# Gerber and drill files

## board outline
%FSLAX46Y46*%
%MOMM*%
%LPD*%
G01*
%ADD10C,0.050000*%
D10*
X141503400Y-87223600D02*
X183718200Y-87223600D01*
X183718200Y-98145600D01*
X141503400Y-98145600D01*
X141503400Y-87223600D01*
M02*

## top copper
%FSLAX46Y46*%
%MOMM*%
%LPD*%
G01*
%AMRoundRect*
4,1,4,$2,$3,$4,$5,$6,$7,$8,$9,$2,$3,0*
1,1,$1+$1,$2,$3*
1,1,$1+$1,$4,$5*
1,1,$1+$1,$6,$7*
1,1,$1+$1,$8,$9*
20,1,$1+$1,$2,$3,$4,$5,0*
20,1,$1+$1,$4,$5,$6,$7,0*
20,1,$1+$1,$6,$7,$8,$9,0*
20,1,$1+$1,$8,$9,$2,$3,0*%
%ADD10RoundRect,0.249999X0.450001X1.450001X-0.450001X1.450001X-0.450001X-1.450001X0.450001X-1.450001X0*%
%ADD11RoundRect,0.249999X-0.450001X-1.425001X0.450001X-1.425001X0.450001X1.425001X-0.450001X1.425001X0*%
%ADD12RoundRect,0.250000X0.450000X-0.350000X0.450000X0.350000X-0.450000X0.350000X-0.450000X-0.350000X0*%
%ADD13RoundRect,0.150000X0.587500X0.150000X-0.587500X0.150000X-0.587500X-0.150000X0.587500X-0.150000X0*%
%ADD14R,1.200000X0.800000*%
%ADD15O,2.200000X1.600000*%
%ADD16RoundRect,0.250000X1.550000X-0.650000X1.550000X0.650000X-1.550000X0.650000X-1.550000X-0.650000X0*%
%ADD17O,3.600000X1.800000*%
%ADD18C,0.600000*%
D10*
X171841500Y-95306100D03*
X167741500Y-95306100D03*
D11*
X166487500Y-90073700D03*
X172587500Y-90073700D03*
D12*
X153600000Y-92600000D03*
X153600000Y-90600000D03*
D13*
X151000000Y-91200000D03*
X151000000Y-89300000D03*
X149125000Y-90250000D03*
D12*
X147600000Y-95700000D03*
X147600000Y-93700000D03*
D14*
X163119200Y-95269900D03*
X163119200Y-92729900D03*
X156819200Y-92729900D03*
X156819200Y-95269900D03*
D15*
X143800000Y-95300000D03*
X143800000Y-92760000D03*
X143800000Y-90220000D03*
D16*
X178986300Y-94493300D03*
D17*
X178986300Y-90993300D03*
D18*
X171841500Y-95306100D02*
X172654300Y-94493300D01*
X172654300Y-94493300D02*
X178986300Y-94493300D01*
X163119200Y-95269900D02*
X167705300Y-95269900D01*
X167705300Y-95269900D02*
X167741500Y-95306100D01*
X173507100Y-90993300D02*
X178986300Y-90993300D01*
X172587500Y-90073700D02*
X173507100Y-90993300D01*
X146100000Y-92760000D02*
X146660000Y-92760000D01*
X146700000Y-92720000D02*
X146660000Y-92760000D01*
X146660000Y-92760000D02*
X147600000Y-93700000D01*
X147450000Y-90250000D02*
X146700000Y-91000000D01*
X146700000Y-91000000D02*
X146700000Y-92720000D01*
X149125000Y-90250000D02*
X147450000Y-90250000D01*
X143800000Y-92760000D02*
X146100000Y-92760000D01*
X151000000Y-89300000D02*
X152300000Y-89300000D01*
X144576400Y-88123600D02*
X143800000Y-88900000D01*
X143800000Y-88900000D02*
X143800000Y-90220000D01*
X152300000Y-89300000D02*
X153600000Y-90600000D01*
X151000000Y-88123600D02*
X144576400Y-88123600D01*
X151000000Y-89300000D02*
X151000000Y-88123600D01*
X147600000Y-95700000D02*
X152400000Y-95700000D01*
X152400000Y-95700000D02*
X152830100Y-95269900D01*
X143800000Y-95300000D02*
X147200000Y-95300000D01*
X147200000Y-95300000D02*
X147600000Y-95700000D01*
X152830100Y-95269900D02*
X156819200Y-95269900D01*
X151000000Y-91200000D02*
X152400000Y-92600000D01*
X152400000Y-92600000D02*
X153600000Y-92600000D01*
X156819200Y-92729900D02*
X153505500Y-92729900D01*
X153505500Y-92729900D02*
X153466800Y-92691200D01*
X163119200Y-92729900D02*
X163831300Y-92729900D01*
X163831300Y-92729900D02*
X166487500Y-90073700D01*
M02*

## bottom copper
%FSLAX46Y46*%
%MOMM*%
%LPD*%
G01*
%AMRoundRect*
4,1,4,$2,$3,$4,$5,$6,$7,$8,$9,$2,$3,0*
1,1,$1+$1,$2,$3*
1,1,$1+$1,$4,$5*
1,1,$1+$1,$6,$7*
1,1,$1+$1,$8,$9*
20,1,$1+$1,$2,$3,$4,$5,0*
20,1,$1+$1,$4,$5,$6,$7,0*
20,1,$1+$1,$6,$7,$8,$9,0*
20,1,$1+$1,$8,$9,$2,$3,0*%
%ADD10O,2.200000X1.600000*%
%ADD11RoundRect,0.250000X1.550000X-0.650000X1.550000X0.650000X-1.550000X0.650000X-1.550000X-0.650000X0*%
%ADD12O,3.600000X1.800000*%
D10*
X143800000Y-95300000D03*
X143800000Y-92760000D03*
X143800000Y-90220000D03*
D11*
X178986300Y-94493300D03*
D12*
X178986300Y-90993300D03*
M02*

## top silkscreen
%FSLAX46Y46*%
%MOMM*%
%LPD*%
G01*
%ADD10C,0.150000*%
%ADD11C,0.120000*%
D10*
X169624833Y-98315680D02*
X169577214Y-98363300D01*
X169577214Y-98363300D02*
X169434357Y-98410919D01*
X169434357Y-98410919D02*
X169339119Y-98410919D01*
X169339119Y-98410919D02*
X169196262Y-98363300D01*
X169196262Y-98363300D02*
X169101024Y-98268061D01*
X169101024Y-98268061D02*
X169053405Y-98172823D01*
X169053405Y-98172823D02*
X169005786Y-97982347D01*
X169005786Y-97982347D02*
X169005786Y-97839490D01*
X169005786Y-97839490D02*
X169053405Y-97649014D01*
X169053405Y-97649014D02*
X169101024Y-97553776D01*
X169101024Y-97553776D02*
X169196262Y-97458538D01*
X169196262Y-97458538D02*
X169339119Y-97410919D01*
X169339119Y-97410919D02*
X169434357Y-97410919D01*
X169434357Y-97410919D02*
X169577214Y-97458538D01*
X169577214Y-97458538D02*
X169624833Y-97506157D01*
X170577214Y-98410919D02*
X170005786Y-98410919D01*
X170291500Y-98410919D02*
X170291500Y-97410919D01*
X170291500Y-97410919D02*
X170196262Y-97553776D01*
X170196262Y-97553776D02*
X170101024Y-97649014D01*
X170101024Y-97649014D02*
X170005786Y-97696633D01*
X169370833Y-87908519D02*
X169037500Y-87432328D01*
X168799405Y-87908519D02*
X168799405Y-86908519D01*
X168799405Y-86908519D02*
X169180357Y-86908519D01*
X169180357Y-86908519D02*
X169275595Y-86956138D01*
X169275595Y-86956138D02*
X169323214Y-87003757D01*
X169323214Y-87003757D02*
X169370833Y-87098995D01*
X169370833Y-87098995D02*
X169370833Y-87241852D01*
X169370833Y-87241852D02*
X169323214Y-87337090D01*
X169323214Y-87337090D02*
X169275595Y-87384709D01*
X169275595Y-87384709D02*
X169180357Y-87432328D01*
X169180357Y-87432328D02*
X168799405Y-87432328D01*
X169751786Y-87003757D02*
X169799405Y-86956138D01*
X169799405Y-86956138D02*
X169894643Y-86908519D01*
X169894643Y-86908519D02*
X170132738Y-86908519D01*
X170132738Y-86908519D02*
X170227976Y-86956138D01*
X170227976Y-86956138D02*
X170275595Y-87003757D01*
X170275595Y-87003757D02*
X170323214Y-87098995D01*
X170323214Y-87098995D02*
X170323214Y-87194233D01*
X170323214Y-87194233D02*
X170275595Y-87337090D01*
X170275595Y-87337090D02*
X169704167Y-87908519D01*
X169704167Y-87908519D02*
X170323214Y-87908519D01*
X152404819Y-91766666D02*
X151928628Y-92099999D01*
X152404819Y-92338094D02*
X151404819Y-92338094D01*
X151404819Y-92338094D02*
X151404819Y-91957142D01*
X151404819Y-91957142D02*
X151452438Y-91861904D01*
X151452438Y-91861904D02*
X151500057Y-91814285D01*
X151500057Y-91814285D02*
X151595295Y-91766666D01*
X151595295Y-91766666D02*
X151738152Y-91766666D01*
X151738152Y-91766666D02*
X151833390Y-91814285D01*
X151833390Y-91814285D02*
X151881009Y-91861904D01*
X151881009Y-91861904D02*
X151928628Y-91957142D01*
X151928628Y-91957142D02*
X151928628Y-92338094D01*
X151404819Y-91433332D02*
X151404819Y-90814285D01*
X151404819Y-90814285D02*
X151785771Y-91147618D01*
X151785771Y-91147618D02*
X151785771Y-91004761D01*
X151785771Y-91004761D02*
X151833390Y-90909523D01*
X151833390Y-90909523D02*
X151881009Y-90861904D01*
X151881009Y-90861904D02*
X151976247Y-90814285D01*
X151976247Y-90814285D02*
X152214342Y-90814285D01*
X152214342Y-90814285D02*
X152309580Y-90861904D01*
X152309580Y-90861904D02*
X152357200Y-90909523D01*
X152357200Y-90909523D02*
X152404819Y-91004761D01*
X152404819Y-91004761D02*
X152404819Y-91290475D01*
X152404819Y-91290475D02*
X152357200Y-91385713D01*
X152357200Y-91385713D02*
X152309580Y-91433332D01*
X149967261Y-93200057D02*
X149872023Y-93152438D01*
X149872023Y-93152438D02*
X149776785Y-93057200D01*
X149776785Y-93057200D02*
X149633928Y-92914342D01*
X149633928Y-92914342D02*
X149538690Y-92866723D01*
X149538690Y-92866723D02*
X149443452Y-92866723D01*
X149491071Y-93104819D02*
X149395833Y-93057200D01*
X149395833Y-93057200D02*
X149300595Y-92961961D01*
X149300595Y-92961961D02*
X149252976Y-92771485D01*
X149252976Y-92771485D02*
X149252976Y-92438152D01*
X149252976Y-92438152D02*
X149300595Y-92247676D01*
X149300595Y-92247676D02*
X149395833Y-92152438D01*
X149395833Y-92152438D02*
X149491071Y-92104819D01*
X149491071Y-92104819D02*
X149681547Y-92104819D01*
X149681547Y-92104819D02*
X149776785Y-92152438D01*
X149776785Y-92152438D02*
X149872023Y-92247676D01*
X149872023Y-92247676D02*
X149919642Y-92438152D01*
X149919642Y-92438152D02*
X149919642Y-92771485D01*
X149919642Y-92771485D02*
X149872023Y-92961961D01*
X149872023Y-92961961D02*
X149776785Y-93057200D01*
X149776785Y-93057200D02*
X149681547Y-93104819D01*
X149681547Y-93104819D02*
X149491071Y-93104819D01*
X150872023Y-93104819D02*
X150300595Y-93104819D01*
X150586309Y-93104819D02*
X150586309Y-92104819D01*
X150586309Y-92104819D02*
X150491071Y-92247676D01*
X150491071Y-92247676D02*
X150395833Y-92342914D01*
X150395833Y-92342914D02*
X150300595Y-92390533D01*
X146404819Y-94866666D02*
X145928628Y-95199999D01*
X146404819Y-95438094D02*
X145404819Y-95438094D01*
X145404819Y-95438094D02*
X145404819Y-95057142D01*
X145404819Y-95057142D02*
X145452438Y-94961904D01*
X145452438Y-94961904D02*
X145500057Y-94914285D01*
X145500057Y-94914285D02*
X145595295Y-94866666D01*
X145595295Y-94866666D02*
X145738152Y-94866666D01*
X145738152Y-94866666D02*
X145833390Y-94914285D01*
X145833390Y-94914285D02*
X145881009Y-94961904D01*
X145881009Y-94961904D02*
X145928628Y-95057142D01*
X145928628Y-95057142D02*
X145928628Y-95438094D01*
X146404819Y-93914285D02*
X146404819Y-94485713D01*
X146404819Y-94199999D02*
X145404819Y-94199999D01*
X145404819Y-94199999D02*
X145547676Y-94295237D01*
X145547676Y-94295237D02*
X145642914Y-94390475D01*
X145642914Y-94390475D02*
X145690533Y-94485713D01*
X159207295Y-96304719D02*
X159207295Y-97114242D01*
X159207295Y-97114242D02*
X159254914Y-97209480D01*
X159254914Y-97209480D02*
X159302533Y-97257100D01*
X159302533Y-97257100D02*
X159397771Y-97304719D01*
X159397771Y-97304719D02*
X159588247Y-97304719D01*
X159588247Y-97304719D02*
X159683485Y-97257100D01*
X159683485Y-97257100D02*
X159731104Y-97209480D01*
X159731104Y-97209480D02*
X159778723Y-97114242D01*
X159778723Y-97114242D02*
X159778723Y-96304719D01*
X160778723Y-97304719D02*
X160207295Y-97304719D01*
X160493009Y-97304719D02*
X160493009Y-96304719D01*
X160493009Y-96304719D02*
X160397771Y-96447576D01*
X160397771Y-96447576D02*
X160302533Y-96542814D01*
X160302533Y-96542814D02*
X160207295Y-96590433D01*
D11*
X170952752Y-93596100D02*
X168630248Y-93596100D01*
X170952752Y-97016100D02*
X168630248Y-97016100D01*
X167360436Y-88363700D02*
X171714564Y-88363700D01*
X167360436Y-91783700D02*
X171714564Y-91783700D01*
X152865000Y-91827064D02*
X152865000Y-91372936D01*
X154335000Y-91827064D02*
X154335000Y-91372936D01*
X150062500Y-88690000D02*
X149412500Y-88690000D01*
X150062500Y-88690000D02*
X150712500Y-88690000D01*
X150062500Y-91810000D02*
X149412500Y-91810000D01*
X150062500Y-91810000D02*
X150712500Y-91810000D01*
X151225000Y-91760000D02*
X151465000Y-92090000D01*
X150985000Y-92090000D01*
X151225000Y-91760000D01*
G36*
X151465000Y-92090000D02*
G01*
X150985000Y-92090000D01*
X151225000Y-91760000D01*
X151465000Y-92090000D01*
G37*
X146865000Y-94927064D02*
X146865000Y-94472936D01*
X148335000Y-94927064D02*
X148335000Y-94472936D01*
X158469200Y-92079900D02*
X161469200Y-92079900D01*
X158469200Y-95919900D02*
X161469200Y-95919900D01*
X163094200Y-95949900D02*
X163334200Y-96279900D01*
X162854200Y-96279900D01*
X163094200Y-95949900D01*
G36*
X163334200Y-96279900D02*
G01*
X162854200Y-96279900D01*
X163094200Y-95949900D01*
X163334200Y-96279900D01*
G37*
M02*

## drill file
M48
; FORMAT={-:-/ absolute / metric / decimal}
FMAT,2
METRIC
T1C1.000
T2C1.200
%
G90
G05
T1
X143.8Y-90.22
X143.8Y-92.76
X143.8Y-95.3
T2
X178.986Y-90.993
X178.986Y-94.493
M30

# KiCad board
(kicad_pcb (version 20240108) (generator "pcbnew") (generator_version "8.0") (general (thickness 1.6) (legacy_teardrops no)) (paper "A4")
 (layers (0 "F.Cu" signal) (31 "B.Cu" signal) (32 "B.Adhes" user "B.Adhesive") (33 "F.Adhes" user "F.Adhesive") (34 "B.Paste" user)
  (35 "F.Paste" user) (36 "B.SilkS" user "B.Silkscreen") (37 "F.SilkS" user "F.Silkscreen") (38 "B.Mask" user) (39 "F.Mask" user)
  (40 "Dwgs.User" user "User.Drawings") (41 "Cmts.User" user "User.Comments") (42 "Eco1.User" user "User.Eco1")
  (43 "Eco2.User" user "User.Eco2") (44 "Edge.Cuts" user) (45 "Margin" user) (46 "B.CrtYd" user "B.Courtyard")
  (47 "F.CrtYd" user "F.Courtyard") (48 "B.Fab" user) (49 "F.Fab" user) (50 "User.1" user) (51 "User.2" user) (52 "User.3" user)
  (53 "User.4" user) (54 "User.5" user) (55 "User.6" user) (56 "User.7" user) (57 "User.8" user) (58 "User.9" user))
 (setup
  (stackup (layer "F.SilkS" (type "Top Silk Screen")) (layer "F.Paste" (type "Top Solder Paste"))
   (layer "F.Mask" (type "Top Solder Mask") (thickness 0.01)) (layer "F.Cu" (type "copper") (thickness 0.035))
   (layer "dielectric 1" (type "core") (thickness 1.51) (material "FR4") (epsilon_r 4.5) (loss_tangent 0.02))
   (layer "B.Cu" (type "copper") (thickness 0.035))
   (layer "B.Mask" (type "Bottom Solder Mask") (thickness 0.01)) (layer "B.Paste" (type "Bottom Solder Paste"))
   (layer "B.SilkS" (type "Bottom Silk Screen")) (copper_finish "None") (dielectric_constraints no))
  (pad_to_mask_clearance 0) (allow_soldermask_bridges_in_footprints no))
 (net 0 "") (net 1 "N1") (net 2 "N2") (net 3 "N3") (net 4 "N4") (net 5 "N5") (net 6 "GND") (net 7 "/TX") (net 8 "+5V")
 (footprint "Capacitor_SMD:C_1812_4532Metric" (layer "F.Cu") (at 169.7915 95.3061 180)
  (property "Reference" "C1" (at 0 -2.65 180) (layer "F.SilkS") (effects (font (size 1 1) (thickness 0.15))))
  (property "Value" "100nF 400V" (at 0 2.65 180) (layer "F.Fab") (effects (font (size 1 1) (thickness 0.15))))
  (fp_line (start -1.161252 1.71) (end 1.161252 1.71) (stroke (width 0.12) (type solid)) (layer "F.SilkS"))
  (fp_line (start -1.161252 -1.71) (end 1.161252 -1.71) (stroke (width 0.12) (type solid)) (layer "F.SilkS"))
  (pad "1" smd roundrect (at -2.05 0 180) (size 1.4 3.4) (layers "F.Cu" "F.Paste" "F.Mask") (roundrect_rratio 0.178571) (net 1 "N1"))
  (pad "2" smd roundrect (at 2.05 0 180) (size 1.4 3.4) (layers "F.Cu" "F.Paste" "F.Mask") (roundrect_rratio 0.178571) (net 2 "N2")))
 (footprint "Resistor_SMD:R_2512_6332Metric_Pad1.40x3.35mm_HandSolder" (layer "F.Cu") (at 169.5375 90.0737)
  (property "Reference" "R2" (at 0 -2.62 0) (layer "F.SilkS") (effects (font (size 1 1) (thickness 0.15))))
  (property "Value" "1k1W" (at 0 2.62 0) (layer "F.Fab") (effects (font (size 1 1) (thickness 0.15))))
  (fp_line (start -2.177064 -1.71) (end 2.177064 -1.71) (stroke (width 0.12) (type solid)) (layer "F.SilkS"))
  (fp_line (start -2.177064 1.71) (end 2.177064 1.71) (stroke (width 0.12) (type solid)) (layer "F.SilkS"))
  (pad "1" smd roundrect (at -3.05 0) (size 1.4 3.35) (layers "F.Cu" "F.Paste" "F.Mask") (roundrect_rratio 0.178571) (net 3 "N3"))
  (pad "2" smd roundrect (at 3.05 0) (size 1.4 3.35) (layers "F.Cu" "F.Paste" "F.Mask") (roundrect_rratio 0.178571) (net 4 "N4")))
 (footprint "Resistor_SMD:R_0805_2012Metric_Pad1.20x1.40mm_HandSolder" (layer "F.Cu") (at 153.6 91.6 90)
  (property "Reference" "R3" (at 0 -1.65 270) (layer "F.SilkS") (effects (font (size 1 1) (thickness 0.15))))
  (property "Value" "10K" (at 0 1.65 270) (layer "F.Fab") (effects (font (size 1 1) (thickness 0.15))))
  (fp_line (start -0.227064 -0.735) (end 0.227064 -0.735) (stroke (width 0.12) (type solid)) (layer "F.SilkS"))
  (fp_line (start -0.227064 0.735) (end 0.227064 0.735) (stroke (width 0.12) (type solid)) (layer "F.SilkS"))
  (pad "1" smd roundrect (at -1 0 90) (size 1.2 1.4) (layers "F.Cu" "F.Paste" "F.Mask") (roundrect_rratio 0.208333) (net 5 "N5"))
  (pad "2" smd roundrect (at 1 0 90) (size 1.2 1.4) (layers "F.Cu" "F.Paste" "F.Mask") (roundrect_rratio 0.208333) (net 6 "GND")))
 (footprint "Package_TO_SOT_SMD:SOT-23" (layer "F.Cu") (at 150.0625 90.25 180)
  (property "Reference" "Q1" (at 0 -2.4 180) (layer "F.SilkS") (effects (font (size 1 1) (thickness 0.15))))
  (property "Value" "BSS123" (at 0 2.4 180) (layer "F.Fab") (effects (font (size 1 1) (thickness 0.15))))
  (fp_line (start 0 1.56) (end 0.65 1.56) (stroke (width 0.12) (type solid)) (layer "F.SilkS"))
  (fp_line (start 0 1.56) (end -0.65 1.56) (stroke (width 0.12) (type solid)) (layer "F.SilkS"))
  (fp_line (start 0 -1.56) (end 0.65 -1.56) (stroke (width 0.12) (type solid)) (layer "F.SilkS"))
  (fp_line (start 0 -1.56) (end -0.65 -1.56) (stroke (width 0.12) (type solid)) (layer "F.SilkS"))
  (fp_poly
   (pts (xy -1.1625 -1.51) (xy -1.4025 -1.84) (xy -0.9225 -1.84) (xy -1.1625 -1.51)) (stroke (width 0.12) (type solid)) (fill solid)
   (layer "F.SilkS"))
  (pad "1" smd roundrect (at -0.9375 -0.95 180) (size 1.475 0.6) (layers "F.Cu" "F.Paste" "F.Mask") (roundrect_rratio 0.25) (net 5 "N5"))
  (pad "2" smd roundrect (at -0.9375 0.95 180) (size 1.475 0.6) (layers "F.Cu" "F.Paste" "F.Mask") (roundrect_rratio 0.25) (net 6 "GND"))
  (pad "3" smd roundrect (at 0.9375 0 180) (size 1.475 0.6) (layers "F.Cu" "F.Paste" "F.Mask") (roundrect_rratio 0.25) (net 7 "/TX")))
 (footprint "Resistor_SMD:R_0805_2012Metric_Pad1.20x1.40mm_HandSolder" (layer "F.Cu") (at 147.6 94.7 90)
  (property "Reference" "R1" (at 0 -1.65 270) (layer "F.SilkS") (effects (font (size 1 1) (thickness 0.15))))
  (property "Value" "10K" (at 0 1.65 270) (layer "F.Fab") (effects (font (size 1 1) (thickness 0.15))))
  (fp_line (start -0.227064 -0.735) (end 0.227064 -0.735) (stroke (width 0.12) (type solid)) (layer "F.SilkS"))
  (fp_line (start -0.227064 0.735) (end 0.227064 0.735) (stroke (width 0.12) (type solid)) (layer "F.SilkS"))
  (pad "1" smd roundrect (at -1 0 90) (size 1.2 1.4) (layers "F.Cu" "F.Paste" "F.Mask") (roundrect_rratio 0.208333) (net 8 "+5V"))
  (pad "2" smd roundrect (at 1 0 90) (size 1.2 1.4) (layers "F.Cu" "F.Paste" "F.Mask") (roundrect_rratio 0.208333) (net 7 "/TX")))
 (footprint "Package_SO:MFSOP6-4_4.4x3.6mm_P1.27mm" (layer "F.Cu") (at 159.9692 93.9999 180)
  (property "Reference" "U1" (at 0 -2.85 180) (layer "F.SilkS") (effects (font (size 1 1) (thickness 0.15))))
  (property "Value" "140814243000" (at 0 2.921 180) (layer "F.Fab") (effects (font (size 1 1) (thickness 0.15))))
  (fp_line (start 1.5 1.92) (end -1.5 1.92) (stroke (width 0.12) (type solid)) (layer "F.SilkS"))
  (fp_line (start 1.5 -1.92) (end -1.5 -1.92) (stroke (width 0.12) (type solid)) (layer "F.SilkS"))
  (fp_poly
   (pts (xy -3.125 -1.95) (xy -3.365 -2.28) (xy -2.885 -2.28) (xy -3.125 -1.95)) (stroke (width 0.12) (type solid)) (fill solid)
   (layer "F.SilkS"))
  (pad "1" smd rect (at -3.15 -1.27 180) (size 1.2 0.8) (layers "F.Cu" "F.Paste" "F.Mask") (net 2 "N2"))
  (pad "3" smd rect (at -3.15 1.27 180) (size 1.2 0.8) (layers "F.Cu" "F.Paste" "F.Mask") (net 3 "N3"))
  (pad "4" smd rect (at 3.15 1.27 180) (size 1.2 0.8) (layers "F.Cu" "F.Paste" "F.Mask") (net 5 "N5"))
  (pad "6" smd rect (at 3.15 -1.27 180) (size 1.2 0.8) (layers "F.Cu" "F.Paste" "F.Mask") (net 8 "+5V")))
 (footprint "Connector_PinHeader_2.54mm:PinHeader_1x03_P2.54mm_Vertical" (layer "B.Cu") (at 143.8 95.3)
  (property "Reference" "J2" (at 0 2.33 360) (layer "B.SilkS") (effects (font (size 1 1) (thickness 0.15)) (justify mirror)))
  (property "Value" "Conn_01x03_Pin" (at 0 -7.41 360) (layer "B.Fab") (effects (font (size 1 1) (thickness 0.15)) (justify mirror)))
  (pad "1" thru_hole oval (at 0 0) (size 2.2 1.6) (drill 1) (layers "*.Cu" "*.Mask") (remove_unused_layers no) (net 8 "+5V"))
  (pad "2" thru_hole oval (at 0 -2.54) (size 2.2 1.6) (drill 1) (layers "*.Cu" "*.Mask") (remove_unused_layers no) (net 7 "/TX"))
  (pad "3" thru_hole oval (at 0 -5.08) (size 2.2 1.6) (drill 1) (layers "*.Cu" "*.Mask") (remove_unused_layers no) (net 6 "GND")))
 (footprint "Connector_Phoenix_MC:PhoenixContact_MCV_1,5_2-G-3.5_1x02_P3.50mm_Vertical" (layer "B.Cu") (at 178.9863 94.4933 90)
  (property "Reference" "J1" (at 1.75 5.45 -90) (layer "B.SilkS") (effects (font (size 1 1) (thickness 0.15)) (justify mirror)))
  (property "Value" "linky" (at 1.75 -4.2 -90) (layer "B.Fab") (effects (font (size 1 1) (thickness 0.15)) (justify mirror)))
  (pad "1" thru_hole roundrect (at 0 0 90) (size 1.8 3.6) (drill 1.2) (layers "*.Cu" "*.Mask") (remove_unused_layers no)
   (roundrect_rratio 0.138889) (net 1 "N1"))
  (pad "2" thru_hole oval (at 3.5 0 90) (size 1.8 3.6) (drill 1.2) (layers "*.Cu" "*.Mask") (remove_unused_layers no) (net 4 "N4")))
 (gr_rect (start 141.5034 87.2236) (end 183.7182 98.1456) (stroke (width 0.05) (type default)) (fill none) (layer "Edge.Cuts"))
 (segment (start 171.8415 95.3061) (end 172.6543 94.4933) (width 0.6) (layer "F.Cu") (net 1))
 (segment (start 172.6543 94.4933) (end 178.9863 94.4933) (width 0.6) (layer "F.Cu") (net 1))
 (segment (start 163.1192 95.2699) (end 167.7053 95.2699) (width 0.6) (layer "F.Cu") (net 2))
 (segment (start 167.7053 95.2699) (end 167.7415 95.3061) (width 0.6) (layer "F.Cu") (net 2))
 (segment (start 173.5071 90.9933) (end 178.9863 90.9933) (width 0.6) (layer "F.Cu") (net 4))
 (segment (start 172.5875 90.0737) (end 173.5071 90.9933) (width 0.6) (layer "F.Cu") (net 4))
 (segment (start 146.1 92.76) (end 146.66 92.76) (width 0.6) (layer "F.Cu") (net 7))
 (segment (start 146.7 92.72) (end 146.66 92.76) (width 0.6) (layer "F.Cu") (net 7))
 (segment (start 146.66 92.76) (end 147.6 93.7) (width 0.6) (layer "F.Cu") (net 7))
 (segment (start 147.45 90.25) (end 146.7 91) (width 0.6) (layer "F.Cu") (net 7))
 (segment (start 146.7 91) (end 146.7 92.72) (width 0.6) (layer "F.Cu") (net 7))
 (segment (start 149.125 90.25) (end 147.45 90.25) (width 0.6) (layer "F.Cu") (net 7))
 (segment (start 143.8 92.76) (end 146.1 92.76) (width 0.6) (layer "F.Cu") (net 7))
 (segment (start 151 89.3) (end 152.3 89.3) (width 0.6) (layer "F.Cu") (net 6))
 (segment (start 144.5764 88.1236) (end 143.8 88.9) (width 0.6) (layer "F.Cu") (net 6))
 (segment (start 143.8 88.9) (end 143.8 90.22) (width 0.6) (layer "F.Cu") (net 6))
 (segment (start 152.3 89.3) (end 153.6 90.6) (width 0.6) (layer "F.Cu") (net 6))
 (segment (start 151 88.1236) (end 144.5764 88.1236) (width 0.6) (layer "F.Cu") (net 6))
 (segment (start 151 89.3) (end 151 88.1236) (width 0.6) (layer "F.Cu") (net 6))
 (segment (start 147.6 95.7) (end 152.4 95.7) (width 0.6) (layer "F.Cu") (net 8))
 (segment (start 152.4 95.7) (end 152.8301 95.2699) (width 0.6) (layer "F.Cu") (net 8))
 (segment (start 143.8 95.3) (end 147.2 95.3) (width 0.6) (layer "F.Cu") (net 8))
 (segment (start 147.2 95.3) (end 147.6 95.7) (width 0.6) (layer "F.Cu") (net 8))
 (segment (start 152.8301 95.2699) (end 156.8192 95.2699) (width 0.6) (layer "F.Cu") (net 8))
 (segment (start 151 91.2) (end 152.4 92.6) (width 0.6) (layer "F.Cu") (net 5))
 (segment (start 152.4 92.6) (end 153.6 92.6) (width 0.6) (layer "F.Cu") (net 5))
 (segment (start 156.8192 92.7299) (end 153.5055 92.7299) (width 0.6) (layer "F.Cu") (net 5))
 (segment (start 153.5055 92.7299) (end 153.4668 92.6912) (width 0.6) (layer "F.Cu") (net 5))
 (segment (start 163.1192 92.7299) (end 163.8313 92.7299) (width 0.6) (layer "F.Cu") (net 3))
 (segment (start 163.8313 92.7299) (end 166.4875 90.0737) (width 0.6) (layer "F.Cu") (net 3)))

